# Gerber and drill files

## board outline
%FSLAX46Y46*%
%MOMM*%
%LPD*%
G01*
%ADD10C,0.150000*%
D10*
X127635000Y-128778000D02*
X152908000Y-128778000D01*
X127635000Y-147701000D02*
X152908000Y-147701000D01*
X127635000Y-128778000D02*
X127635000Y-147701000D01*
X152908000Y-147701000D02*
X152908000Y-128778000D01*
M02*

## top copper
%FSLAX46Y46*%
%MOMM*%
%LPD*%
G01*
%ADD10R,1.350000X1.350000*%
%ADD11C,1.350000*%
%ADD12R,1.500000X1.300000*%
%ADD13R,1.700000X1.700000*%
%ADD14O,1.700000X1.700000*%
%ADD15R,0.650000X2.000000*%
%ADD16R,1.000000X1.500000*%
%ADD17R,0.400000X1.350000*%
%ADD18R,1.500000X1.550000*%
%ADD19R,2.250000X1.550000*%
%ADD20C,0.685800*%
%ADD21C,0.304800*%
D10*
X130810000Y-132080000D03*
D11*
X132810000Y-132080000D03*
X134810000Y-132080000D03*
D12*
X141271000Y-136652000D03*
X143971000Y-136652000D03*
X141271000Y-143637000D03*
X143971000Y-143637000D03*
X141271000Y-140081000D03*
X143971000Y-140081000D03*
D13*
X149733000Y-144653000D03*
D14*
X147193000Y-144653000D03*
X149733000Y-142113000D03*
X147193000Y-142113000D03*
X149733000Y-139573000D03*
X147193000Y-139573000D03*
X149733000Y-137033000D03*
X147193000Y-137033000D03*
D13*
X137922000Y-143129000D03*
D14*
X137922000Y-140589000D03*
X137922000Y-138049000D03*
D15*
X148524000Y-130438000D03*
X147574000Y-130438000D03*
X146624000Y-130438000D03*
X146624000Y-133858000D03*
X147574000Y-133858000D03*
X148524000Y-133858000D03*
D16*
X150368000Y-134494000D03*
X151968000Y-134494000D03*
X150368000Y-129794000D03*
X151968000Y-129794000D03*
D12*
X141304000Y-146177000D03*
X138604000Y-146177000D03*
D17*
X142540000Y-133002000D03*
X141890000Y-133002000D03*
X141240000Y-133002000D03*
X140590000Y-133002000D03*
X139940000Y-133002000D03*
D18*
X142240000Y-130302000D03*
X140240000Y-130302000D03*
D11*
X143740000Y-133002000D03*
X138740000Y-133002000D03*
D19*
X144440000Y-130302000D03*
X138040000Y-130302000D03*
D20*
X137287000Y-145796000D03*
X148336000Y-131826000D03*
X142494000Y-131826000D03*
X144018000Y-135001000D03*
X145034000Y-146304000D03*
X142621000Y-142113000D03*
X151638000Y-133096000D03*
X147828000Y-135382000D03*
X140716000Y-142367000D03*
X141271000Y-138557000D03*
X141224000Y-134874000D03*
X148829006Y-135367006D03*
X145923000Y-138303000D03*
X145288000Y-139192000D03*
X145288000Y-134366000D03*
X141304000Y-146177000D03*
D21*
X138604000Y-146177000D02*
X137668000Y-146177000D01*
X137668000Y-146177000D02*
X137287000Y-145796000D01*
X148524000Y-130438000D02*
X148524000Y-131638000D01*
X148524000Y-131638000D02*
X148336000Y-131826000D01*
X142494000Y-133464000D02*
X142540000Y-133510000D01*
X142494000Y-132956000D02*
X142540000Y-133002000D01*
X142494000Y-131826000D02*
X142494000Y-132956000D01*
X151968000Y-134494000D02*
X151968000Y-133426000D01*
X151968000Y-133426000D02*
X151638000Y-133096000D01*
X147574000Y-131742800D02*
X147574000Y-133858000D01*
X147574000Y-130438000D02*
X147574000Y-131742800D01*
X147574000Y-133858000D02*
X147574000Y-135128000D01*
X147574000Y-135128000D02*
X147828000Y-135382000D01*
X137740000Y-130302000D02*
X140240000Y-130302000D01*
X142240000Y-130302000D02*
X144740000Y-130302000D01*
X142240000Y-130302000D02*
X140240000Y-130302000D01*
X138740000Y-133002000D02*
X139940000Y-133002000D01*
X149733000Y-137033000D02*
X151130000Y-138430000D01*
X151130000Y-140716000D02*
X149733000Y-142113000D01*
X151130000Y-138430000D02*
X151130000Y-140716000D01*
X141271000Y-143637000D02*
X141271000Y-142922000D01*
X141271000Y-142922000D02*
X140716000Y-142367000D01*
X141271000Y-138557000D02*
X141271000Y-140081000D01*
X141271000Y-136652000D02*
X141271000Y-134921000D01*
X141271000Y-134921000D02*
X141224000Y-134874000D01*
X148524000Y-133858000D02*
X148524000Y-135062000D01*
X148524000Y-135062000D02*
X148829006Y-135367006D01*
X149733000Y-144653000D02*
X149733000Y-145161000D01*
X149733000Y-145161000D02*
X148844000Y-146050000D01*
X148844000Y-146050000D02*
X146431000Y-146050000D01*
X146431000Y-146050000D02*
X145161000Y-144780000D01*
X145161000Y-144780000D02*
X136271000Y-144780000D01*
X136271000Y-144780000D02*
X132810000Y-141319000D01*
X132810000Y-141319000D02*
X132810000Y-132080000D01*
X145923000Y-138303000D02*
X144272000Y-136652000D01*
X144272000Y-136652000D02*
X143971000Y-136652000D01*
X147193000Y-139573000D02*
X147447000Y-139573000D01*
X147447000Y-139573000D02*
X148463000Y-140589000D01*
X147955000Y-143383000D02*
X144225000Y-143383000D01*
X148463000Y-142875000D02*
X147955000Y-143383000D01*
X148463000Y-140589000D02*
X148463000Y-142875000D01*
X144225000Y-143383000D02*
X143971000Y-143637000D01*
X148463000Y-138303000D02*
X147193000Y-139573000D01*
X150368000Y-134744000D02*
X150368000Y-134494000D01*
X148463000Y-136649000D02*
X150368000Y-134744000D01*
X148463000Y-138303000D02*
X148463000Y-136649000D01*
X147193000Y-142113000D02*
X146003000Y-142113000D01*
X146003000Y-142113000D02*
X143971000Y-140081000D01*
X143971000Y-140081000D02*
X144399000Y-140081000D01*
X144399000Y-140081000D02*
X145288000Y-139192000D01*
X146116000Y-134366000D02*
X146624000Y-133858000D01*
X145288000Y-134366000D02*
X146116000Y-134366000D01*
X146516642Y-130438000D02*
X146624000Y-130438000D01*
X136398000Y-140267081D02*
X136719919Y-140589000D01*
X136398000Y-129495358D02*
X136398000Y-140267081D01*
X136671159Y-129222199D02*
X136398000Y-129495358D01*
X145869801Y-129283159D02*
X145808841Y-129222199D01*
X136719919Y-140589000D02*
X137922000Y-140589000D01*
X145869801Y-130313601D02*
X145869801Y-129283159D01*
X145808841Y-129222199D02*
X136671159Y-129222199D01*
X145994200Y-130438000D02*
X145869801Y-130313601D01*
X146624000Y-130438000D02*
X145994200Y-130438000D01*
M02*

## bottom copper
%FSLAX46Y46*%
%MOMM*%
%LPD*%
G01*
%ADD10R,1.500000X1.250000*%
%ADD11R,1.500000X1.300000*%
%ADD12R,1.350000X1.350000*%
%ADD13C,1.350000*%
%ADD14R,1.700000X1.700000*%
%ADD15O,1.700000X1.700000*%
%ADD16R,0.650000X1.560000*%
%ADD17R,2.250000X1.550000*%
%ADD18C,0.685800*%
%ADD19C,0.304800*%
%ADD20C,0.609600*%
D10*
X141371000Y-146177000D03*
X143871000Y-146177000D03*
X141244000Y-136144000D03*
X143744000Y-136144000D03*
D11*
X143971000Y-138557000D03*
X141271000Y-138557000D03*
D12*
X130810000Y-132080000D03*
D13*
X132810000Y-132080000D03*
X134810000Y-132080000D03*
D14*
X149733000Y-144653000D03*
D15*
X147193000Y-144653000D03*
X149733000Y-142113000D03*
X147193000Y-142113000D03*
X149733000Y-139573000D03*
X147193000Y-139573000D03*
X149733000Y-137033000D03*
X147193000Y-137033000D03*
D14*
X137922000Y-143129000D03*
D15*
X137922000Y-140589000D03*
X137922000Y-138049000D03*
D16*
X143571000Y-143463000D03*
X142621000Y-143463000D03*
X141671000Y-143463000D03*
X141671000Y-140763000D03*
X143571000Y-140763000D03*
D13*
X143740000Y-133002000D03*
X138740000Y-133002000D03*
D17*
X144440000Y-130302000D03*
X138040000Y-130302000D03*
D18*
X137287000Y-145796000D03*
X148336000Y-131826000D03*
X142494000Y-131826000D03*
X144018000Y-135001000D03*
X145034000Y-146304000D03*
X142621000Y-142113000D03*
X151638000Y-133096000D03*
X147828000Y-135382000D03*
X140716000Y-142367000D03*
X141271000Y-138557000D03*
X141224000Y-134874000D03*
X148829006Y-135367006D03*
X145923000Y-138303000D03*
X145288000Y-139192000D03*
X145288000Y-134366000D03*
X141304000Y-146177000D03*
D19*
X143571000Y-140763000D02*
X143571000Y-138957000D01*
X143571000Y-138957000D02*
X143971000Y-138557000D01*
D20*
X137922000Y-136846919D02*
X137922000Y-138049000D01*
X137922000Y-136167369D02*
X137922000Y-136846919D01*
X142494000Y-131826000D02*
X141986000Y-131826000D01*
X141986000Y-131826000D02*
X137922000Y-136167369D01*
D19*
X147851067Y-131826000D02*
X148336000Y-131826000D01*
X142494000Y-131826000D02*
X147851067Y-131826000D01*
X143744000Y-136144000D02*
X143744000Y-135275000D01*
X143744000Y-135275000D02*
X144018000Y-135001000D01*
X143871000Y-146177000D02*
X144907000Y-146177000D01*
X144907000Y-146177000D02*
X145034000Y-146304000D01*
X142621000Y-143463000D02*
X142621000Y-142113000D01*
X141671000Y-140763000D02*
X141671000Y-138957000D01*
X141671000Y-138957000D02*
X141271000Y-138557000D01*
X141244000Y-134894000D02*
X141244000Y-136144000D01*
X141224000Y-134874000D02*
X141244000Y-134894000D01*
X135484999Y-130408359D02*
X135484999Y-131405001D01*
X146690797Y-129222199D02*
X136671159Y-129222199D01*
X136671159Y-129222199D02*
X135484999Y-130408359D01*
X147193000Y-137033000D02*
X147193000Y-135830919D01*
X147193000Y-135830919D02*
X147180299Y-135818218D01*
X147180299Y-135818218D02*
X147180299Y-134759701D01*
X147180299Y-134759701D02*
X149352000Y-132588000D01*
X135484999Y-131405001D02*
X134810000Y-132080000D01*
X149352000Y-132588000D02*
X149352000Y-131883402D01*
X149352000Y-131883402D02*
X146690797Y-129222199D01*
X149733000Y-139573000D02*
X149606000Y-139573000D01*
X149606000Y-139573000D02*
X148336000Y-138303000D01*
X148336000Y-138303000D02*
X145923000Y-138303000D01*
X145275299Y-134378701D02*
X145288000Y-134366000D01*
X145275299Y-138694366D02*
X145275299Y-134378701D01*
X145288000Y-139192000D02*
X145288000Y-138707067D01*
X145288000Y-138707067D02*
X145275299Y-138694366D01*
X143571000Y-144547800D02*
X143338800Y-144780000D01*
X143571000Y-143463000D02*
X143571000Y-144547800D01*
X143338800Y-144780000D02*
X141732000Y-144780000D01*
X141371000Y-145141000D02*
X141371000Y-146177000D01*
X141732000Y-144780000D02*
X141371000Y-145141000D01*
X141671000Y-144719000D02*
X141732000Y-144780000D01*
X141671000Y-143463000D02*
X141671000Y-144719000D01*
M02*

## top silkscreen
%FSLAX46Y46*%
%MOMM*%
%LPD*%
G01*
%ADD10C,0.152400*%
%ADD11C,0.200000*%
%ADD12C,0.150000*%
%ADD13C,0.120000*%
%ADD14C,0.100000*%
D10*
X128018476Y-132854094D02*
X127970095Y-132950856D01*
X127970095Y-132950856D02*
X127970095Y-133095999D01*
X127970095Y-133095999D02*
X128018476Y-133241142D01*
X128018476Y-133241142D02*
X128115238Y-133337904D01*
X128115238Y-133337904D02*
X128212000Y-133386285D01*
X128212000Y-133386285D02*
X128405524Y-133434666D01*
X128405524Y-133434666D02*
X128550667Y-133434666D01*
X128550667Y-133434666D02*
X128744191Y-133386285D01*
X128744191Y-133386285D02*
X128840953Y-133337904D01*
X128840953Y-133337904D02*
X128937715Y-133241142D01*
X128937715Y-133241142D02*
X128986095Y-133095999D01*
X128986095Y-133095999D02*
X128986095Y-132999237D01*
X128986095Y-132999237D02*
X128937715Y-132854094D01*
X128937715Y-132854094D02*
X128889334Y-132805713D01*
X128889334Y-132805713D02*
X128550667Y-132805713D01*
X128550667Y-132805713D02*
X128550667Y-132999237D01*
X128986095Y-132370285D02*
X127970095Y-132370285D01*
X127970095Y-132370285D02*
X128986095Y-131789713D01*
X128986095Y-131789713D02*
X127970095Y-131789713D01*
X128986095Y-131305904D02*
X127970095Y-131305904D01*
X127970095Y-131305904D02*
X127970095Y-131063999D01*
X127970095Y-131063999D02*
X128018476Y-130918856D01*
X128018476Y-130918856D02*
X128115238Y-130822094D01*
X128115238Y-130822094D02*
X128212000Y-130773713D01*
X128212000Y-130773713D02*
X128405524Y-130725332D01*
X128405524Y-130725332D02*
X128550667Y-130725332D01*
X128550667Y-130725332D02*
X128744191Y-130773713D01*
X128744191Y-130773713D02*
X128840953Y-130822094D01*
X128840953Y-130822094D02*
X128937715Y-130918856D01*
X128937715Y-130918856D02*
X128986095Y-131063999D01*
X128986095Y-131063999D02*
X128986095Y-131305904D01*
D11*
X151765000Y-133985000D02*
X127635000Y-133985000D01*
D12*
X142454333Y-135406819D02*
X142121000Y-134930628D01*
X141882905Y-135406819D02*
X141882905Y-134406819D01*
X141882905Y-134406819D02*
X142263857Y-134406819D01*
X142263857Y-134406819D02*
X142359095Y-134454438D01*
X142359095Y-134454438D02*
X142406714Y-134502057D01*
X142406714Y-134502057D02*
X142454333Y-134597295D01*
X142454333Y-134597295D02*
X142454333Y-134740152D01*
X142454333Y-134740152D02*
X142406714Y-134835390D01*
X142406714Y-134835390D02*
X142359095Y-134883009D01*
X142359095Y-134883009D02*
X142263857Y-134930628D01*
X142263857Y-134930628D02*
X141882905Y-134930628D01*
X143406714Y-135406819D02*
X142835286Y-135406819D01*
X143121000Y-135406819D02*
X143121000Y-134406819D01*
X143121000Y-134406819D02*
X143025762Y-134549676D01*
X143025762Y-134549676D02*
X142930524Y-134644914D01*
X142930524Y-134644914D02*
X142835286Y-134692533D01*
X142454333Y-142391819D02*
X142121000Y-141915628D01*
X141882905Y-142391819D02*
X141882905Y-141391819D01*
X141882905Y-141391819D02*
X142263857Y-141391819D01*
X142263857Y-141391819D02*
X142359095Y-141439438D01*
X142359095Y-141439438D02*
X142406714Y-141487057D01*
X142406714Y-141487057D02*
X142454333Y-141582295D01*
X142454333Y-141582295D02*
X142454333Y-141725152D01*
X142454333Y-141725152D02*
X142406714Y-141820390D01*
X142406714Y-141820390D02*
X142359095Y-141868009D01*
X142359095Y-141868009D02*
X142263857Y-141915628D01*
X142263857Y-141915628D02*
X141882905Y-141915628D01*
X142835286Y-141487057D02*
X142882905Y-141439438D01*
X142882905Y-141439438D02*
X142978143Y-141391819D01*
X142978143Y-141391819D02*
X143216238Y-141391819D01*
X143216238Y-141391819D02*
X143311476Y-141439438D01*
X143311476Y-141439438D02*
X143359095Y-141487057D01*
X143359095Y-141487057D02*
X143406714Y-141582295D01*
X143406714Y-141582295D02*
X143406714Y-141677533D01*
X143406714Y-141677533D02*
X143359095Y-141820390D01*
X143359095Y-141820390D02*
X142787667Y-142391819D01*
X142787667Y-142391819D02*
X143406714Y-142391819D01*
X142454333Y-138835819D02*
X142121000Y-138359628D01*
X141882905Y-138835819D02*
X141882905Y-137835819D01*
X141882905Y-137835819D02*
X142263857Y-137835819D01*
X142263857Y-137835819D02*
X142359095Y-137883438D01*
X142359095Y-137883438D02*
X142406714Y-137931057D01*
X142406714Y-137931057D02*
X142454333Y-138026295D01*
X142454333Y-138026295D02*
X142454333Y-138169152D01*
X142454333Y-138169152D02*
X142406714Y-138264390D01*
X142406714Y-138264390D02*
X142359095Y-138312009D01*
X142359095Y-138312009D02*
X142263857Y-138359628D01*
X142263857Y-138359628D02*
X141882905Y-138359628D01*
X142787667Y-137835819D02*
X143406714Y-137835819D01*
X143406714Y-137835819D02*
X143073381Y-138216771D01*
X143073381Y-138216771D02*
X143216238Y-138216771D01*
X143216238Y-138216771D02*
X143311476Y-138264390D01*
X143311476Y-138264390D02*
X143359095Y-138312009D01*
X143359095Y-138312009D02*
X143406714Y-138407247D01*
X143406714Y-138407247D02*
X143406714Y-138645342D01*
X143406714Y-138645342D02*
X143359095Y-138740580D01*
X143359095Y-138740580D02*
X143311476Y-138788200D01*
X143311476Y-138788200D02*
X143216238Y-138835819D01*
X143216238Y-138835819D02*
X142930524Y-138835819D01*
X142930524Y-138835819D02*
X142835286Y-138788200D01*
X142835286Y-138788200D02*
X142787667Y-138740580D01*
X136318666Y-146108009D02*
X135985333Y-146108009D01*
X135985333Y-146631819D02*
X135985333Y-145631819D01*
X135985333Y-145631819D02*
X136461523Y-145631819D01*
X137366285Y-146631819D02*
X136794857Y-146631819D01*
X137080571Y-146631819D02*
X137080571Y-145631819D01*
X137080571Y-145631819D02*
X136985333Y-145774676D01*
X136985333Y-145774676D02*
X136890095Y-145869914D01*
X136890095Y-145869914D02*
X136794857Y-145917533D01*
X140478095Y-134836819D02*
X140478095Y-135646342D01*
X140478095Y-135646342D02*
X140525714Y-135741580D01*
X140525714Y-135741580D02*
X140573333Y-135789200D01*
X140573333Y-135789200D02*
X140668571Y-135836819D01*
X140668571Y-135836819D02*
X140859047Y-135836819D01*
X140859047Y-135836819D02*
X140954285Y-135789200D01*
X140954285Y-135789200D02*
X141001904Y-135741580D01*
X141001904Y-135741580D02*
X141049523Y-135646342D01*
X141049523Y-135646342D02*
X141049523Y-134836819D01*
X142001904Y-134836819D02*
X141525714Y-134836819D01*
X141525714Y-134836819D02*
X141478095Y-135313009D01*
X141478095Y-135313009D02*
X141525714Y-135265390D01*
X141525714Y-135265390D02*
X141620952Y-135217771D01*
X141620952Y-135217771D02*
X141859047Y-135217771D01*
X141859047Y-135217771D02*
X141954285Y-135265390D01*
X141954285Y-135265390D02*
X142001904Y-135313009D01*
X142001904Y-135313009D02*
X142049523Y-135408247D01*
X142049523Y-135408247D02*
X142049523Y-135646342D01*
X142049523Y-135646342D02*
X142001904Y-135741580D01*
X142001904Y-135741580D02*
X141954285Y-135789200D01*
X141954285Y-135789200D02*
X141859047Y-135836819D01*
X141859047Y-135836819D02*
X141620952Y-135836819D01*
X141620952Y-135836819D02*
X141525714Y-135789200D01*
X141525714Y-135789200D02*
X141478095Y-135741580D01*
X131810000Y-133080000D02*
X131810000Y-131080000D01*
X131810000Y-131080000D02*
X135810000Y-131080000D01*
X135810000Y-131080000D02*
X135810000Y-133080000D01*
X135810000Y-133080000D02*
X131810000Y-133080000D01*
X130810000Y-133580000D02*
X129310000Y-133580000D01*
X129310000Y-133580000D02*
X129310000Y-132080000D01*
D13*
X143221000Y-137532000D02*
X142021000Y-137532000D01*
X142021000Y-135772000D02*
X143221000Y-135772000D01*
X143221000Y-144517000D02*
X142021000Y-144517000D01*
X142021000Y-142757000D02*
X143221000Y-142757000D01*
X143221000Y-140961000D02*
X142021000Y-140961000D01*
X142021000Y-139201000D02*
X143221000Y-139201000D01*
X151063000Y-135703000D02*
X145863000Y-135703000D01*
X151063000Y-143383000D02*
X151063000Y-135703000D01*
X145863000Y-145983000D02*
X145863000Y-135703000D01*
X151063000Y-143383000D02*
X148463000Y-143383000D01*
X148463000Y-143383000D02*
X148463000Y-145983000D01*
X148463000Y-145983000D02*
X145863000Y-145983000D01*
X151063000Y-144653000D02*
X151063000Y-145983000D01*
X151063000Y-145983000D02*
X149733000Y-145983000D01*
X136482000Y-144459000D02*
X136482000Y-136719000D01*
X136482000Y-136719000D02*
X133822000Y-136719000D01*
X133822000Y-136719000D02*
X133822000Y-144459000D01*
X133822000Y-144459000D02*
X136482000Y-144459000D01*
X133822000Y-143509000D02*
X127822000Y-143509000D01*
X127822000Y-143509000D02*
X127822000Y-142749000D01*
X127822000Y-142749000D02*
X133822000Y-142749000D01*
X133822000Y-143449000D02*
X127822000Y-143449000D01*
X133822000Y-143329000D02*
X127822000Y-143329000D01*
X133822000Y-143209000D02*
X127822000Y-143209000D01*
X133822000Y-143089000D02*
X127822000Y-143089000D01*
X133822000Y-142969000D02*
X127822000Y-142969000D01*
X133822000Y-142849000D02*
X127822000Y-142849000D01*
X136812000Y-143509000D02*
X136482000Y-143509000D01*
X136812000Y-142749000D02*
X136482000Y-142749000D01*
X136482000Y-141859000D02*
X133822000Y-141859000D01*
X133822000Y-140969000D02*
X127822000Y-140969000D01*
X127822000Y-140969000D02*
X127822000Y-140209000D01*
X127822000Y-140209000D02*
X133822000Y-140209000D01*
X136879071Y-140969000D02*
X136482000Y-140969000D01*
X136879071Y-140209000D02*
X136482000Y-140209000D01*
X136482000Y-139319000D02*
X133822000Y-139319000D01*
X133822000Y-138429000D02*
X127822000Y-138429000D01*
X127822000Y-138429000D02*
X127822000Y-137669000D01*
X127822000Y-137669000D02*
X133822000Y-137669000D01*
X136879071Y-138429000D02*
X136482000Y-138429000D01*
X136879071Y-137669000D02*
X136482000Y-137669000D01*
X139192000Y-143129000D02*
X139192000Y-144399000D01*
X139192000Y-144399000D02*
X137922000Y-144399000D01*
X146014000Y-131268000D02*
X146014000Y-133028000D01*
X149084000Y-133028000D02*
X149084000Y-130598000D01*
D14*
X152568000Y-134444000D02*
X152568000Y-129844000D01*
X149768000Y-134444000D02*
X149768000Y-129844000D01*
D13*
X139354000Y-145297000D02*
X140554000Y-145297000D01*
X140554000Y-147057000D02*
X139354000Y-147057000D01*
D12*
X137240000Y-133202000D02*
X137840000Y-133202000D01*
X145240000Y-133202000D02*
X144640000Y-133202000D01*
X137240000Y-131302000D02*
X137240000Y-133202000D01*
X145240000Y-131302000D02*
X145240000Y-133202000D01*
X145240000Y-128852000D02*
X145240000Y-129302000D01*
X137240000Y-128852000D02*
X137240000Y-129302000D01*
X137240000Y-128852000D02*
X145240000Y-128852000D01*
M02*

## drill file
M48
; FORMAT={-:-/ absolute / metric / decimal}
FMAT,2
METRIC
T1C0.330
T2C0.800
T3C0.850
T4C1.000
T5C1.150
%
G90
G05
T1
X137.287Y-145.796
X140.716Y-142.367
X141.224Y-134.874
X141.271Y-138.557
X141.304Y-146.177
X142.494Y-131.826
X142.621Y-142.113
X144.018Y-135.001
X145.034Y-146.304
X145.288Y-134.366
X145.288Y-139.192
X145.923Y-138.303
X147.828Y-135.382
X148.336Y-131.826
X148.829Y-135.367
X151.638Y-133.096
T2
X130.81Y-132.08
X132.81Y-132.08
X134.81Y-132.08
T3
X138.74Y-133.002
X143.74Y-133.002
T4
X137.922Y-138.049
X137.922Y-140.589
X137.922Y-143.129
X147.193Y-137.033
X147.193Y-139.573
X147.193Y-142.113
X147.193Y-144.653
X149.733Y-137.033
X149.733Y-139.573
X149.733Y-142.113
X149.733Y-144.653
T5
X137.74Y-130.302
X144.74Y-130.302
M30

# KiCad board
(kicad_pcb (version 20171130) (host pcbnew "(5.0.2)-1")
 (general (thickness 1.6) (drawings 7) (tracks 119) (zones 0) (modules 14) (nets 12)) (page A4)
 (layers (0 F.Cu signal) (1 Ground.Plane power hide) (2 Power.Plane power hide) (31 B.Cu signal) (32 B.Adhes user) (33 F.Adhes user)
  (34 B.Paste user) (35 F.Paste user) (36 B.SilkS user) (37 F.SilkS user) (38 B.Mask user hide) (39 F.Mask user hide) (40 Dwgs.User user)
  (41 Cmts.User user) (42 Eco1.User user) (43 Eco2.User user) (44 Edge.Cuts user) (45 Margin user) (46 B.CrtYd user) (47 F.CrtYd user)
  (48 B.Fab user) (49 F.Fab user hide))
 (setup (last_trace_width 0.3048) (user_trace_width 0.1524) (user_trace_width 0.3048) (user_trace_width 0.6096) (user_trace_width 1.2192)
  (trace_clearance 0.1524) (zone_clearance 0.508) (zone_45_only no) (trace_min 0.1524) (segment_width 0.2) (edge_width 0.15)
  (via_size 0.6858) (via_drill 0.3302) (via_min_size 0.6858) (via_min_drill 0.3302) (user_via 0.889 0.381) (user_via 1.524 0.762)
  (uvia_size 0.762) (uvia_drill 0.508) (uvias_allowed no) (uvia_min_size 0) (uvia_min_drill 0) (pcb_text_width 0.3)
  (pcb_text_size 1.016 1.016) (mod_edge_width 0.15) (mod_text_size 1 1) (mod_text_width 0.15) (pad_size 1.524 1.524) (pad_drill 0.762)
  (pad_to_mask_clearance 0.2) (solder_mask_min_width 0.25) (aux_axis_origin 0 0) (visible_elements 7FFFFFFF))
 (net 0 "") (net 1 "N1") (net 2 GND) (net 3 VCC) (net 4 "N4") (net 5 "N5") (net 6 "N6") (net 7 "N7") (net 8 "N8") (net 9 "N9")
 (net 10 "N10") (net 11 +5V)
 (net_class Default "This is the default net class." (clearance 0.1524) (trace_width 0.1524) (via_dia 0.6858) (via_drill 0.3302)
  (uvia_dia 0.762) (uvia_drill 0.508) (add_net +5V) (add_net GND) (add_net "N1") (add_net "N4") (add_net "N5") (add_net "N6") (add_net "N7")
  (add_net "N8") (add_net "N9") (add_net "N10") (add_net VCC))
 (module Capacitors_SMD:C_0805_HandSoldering (layer B.Cu) (at 142.621 146.177)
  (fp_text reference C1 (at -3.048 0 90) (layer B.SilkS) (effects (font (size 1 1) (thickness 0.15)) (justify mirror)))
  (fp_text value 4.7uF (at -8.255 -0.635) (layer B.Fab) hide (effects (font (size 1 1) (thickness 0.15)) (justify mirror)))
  (pad 1 smd rect (at -1.25 0) (size 1.5 1.25) (layers B.Cu B.Paste B.Mask) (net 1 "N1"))
  (pad 2 smd rect (at 1.25 0) (size 1.5 1.25) (layers B.Cu B.Paste B.Mask) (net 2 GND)))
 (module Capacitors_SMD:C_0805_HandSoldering (layer B.Cu) (at 142.494 136.144)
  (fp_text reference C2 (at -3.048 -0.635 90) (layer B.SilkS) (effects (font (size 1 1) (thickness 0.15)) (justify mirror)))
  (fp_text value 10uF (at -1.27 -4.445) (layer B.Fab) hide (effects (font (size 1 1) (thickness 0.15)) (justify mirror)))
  (pad 1 smd rect (at -1.25 0) (size 1.5 1.25) (layers B.Cu B.Paste B.Mask) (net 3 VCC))
  (pad 2 smd rect (at 1.25 0) (size 1.5 1.25) (layers B.Cu B.Paste B.Mask) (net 2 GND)))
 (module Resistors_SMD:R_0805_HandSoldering (layer B.Cu) (at 142.621 138.557 180)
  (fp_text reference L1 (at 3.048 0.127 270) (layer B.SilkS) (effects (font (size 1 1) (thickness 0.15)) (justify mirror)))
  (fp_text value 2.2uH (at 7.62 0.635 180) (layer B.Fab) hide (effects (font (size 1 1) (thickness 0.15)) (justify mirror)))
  (pad 1 smd rect (at -1.35 0 180) (size 1.5 1.3) (layers B.Cu B.Paste B.Mask) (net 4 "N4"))
  (pad 2 smd rect (at 1.35 0 180) (size 1.5 1.3) (layers B.Cu B.Paste B.Mask) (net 3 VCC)))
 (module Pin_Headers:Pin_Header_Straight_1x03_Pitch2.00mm (layer F.Cu) (at 130.81 132.08 90)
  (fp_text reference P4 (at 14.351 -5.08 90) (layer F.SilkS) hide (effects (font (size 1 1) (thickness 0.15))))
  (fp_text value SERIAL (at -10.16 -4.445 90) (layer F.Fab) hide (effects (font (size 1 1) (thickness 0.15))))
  (fp_line (start -1 1) (end 1 1) (layer F.SilkS) (width 0.15)) (fp_line (start 1 1) (end 1 5) (layer F.SilkS) (width 0.15))
  (fp_line (start 1 5) (end -1 5) (layer F.SilkS) (width 0.15))
  (fp_line (start -1 5) (end -1 1) (layer F.SilkS) (width 0.15))
  (fp_line (start -1.5 0) (end -1.5 -1.5) (layer F.SilkS) (width 0.15))
  (fp_line (start -1.5 -1.5) (end 0 -1.5) (layer F.SilkS) (width 0.15))
  (pad 1 thru_hole rect (at 0 0 90) (size 1.35 1.35) (drill 0.8) (layers *.Cu *.Mask) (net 2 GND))
  (pad 2 thru_hole circle (at 0 2 90) (size 1.35 1.35) (drill 0.8) (layers *.Cu *.Mask) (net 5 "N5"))
  (pad 3 thru_hole circle (at 0 4 90) (size 1.35 1.35) (drill 0.8) (layers *.Cu *.Mask) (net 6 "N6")))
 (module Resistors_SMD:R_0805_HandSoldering (layer F.Cu) (at 142.621 136.652)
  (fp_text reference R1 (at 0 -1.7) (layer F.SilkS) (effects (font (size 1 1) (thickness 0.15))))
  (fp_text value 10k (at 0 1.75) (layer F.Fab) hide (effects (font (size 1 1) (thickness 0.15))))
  (fp_line (start 0.6 0.88) (end -0.6 0.88) (layer F.SilkS) (width 0.12))
  (fp_line (start -0.6 -0.88) (end 0.6 -0.88) (layer F.SilkS) (width 0.12))
  (pad 1 smd rect (at -1.35 0) (size 1.5 1.3) (layers F.Cu F.Paste F.Mask) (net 3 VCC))
  (pad 2 smd rect (at 1.35 0) (size 1.5 1.3) (layers F.Cu F.Paste F.Mask) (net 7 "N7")))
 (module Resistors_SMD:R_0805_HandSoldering (layer F.Cu) (at 142.621 143.637)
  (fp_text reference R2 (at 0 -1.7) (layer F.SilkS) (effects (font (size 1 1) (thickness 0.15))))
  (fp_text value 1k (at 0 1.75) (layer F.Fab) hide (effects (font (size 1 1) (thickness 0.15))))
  (fp_line (start 0.6 0.88) (end -0.6 0.88) (layer F.SilkS) (width 0.12))
  (fp_line (start -0.6 -0.88) (end 0.6 -0.88) (layer F.SilkS) (width 0.12))
  (pad 1 smd rect (at -1.35 0) (size 1.5 1.3) (layers F.Cu F.Paste F.Mask) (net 3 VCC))
  (pad 2 smd rect (at 1.35 0) (size 1.5 1.3) (layers F.Cu F.Paste F.Mask) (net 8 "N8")))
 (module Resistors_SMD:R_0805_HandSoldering (layer F.Cu) (at 142.621 140.081)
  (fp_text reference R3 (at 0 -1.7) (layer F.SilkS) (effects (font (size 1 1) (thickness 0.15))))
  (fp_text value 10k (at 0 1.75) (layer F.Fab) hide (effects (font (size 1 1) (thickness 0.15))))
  (fp_line (start 0.6 0.88) (end -0.6 0.88) (layer F.SilkS) (width 0.12))
  (fp_line (start -0.6 -0.88) (end 0.6 -0.88) (layer F.SilkS) (width 0.12))
  (pad 1 smd rect (at -1.35 0) (size 1.5 1.3) (layers F.Cu F.Paste F.Mask) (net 3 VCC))
  (pad 2 smd rect (at 1.35 0) (size 1.5 1.3) (layers F.Cu F.Paste F.Mask) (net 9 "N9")))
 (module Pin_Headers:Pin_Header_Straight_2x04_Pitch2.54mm (layer F.Cu) (at 149.733 144.653 180)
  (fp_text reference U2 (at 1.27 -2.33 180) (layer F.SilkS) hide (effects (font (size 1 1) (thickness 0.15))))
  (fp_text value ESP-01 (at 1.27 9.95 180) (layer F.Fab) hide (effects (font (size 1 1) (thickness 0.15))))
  (fp_line (start -1.33 8.95) (end 3.87 8.95) (layer F.SilkS) (width 0.12))
  (fp_line (start -1.33 1.27) (end -1.33 8.95) (layer F.SilkS) (width 0.12))
  (fp_line (start 3.87 -1.33) (end 3.87 8.95) (layer F.SilkS) (width 0.12))
  (fp_line (start -1.33 1.27) (end 1.27 1.27) (layer F.SilkS) (width 0.12))
  (fp_line (start 1.27 1.27) (end 1.27 -1.33) (layer F.SilkS) (width 0.12))
  (fp_line (start 1.27 -1.33) (end 3.87 -1.33) (layer F.SilkS) (width 0.12))
  (fp_line (start -1.33 0) (end -1.33 -1.33) (layer F.SilkS) (width 0.12))
  (fp_line (start -1.33 -1.33) (end 0 -1.33) (layer F.SilkS) (width 0.12))
  (pad 1 thru_hole rect (at 0 0 180) (size 1.7 1.7) (drill 1) (layers *.Cu *.Mask) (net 5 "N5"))
  (pad 2 thru_hole oval (at 2.54 0 180) (size 1.7 1.7) (drill 1) (layers *.Cu *.Mask) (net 2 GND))
  (pad 3 thru_hole oval (at 0 2.54 180) (size 1.7 1.7) (drill 1) (layers *.Cu *.Mask) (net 3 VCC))
  (pad 4 thru_hole oval (at 2.54 2.54 180) (size 1.7 1.7) (drill 1) (layers *.Cu *.Mask) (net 9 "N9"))
  (pad 5 thru_hole oval (at 0 5.08 180) (size 1.7 1.7) (drill 1) (layers *.Cu *.Mask) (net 7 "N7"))
  (pad 6 thru_hole oval (at 2.54 5.08 180) (size 1.7 1.7) (drill 1) (layers *.Cu *.Mask) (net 8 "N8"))
  (pad 7 thru_hole oval (at 0 7.62 180) (size 1.7 1.7) (drill 1) (layers *.Cu *.Mask) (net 3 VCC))
  (pad 8 thru_hole oval (at 2.54 7.62 180) (size 1.7 1.7) (drill 1) (layers *.Cu *.Mask) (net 6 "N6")))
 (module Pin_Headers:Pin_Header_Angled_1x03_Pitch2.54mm (layer F.Cu) (at 137.922 143.129 180)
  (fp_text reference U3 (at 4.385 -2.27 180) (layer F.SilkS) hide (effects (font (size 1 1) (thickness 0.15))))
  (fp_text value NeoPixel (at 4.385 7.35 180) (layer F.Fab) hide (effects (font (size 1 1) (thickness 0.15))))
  (fp_line (start 1.44 -1.33) (end 1.44 6.41) (layer F.SilkS) (width 0.12))
  (fp_line (start 1.44 6.41) (end 4.1 6.41) (layer F.SilkS) (width 0.12))
  (fp_line (start 4.1 6.41) (end 4.1 -1.33) (layer F.SilkS) (width 0.12))
  (fp_line (start 4.1 -1.33) (end 1.44 -1.33) (layer F.SilkS) (width 0.12))
  (fp_line (start 4.1 -0.38) (end 10.1 -0.38) (layer F.SilkS) (width 0.12))
  (fp_line (start 10.1 -0.38) (end 10.1 0.38) (layer F.SilkS) (width 0.12))
  (fp_line (start 10.1 0.38) (end 4.1 0.38) (layer F.SilkS) (width 0.12))
  (fp_line (start 4.1 -0.32) (end 10.1 -0.32) (layer F.SilkS) (width 0.12))
  (fp_line (start 4.1 -0.2) (end 10.1 -0.2) (layer F.SilkS) (width 0.12))
  (fp_line (start 4.1 -0.08) (end 10.1 -0.08) (layer F.SilkS) (width 0.12))
  (fp_line (start 4.1 0.04) (end 10.1 0.04) (layer F.SilkS) (width 0.12))
  (fp_line (start 4.1 0.16) (end 10.1 0.16) (layer F.SilkS) (width 0.12))
  (fp_line (start 4.1 0.28) (end 10.1 0.28) (layer F.SilkS) (width 0.12))
  (fp_line (start 1.11 -0.38) (end 1.44 -0.38) (layer F.SilkS) (width 0.12))
  (fp_line (start 1.11 0.38) (end 1.44 0.38) (layer F.SilkS) (width 0.12))
  (fp_line (start 1.44 1.27) (end 4.1 1.27) (layer F.SilkS) (width 0.12))
  (fp_line (start 4.1 2.16) (end 10.1 2.16) (layer F.SilkS) (width 0.12))
  (fp_line (start 10.1 2.16) (end 10.1 2.92) (layer F.SilkS) (width 0.12))
  (fp_line (start 10.1 2.92) (end 4.1 2.92) (layer F.SilkS) (width 0.12))
  (fp_line (start 1.042929 2.16) (end 1.44 2.16) (layer F.SilkS) (width 0.12))
  (fp_line (start 1.042929 2.92) (end 1.44 2.92) (layer F.SilkS) (width 0.12))
  (fp_line (start 1.44 3.81) (end 4.1 3.81) (layer F.SilkS) (width 0.12))
  (fp_line (start 4.1 4.7) (end 10.1 4.7) (layer F.SilkS) (width 0.12))
  (fp_line (start 10.1 4.7) (end 10.1 5.46) (layer F.SilkS) (width 0.12))
  (fp_line (start 10.1 5.46) (end 4.1 5.46) (layer F.SilkS) (width 0.12))
  (fp_line (start 1.042929 4.7) (end 1.44 4.7) (layer F.SilkS) (width 0.12))
  (fp_line (start 1.042929 5.46) (end 1.44 5.46) (layer F.SilkS) (width 0.12))
  (fp_line (start -1.27 0) (end -1.27 -1.27) (layer F.SilkS) (width 0.12))
  (fp_line (start -1.27 -1.27) (end 0 -1.27) (layer F.SilkS) (width 0.12))
  (pad 1 thru_hole rect (at 0 0 180) (size 1.7 1.7) (drill 1) (layers *.Cu *.Mask) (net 2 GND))
  (pad 2 thru_hole oval (at 0 2.54 180) (size 1.7 1.7) (drill 1) (layers *.Cu *.Mask) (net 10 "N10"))
  (pad 3 thru_hole oval (at 0 5.08 180) (size 1.7 1.7) (drill 1) (layers *.Cu *.Mask) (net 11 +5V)))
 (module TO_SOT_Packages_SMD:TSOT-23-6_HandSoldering (layer F.Cu) (at 147.574 132.148 270)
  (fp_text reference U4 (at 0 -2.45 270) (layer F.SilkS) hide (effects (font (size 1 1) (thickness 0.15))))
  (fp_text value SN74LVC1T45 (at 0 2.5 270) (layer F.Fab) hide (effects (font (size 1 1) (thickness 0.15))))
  (fp_line (start -0.88 1.56) (end 0.88 1.56) (layer F.SilkS) (width 0.12))
  (fp_line (start 0.88 -1.51) (end -1.55 -1.51) (layer F.SilkS) (width 0.12))
  (pad 1 smd rect (at -1.71 -0.95 270) (size 2 0.65) (layers F.Cu F.Paste F.Mask) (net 11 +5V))
  (pad 2 smd rect (at -1.71 0 270) (size 2 0.65) (layers F.Cu F.Paste F.Mask) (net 2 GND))
  (pad 3 smd rect (at -1.71 0.95 270) (size 2 0.65) (layers F.Cu F.Paste F.Mask) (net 10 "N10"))
  (pad 4 smd rect (at 1.71 0.95 270) (size 2 0.65) (layers F.Cu F.Paste F.Mask) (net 9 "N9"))
  (pad 5 smd rect (at 1.71 0 270) (size 2 0.65) (layers F.Cu F.Paste F.Mask) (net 2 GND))
  (pad 6 smd rect (at 1.71 -0.95 270) (size 2 0.65) (layers F.Cu F.Paste F.Mask) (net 3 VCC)))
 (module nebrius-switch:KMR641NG (layer F.Cu) (at 151.168 132.144 90)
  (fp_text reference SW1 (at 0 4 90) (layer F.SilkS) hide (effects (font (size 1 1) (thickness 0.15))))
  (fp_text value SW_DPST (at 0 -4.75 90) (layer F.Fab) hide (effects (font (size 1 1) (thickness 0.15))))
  (fp_line (start -2.3 1.4) (end 2.3 1.4) (layer F.SilkS) (width 0.1))
  (fp_line (start -2.3 -1.4) (end 2.3 -1.4) (layer F.SilkS) (width 0.1))
  (pad 1 smd rect (at -2.35 -0.8 90) (size 1.5 1) (layers F.Cu F.Paste F.Mask) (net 8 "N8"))
  (pad 2 smd rect (at -2.35 0.8 90) (size 1.5 1) (layers F.Cu F.Paste F.Mask) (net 2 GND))
  (pad 3 smd rect (at 2.35 -0.8 90) (size 1.5 1) (layers F.Cu F.Paste F.Mask))
  (pad 4 smd rect (at 2.35 0.8 90) (size 1.5 1) (layers F.Cu F.Paste F.Mask)))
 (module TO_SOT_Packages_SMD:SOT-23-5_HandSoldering (layer B.Cu) (at 142.621 142.113 90)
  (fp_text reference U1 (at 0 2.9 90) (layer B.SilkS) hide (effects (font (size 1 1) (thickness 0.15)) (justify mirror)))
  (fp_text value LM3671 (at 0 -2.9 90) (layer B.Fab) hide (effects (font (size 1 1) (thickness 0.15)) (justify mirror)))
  (pad 1 smd rect (at -1.35 0.95 90) (size 1.56 0.65) (layers B.Cu B.Paste B.Mask) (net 1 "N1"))
  (pad 2 smd rect (at -1.35 0 90) (size 1.56 0.65) (layers B.Cu B.Paste B.Mask) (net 2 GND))
  (pad 3 smd rect (at -1.35 -0.95 90) (size 1.56 0.65) (layers B.Cu B.Paste B.Mask) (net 1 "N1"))
  (pad 4 smd rect (at 1.35 -0.95 90) (size 1.56 0.65) (layers B.Cu B.Paste B.Mask) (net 3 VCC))
  (pad 5 smd rect (at 1.35 0.95 90) (size 1.56 0.65) (layers B.Cu B.Paste B.Mask) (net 4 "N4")))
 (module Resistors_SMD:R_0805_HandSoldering (layer F.Cu) (at 139.954 146.177 180)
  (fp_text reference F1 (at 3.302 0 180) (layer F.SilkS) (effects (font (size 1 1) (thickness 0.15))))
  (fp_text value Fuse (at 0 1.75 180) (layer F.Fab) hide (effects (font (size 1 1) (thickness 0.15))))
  (fp_line (start 0.6 0.88) (end -0.6 0.88) (layer F.SilkS) (width 0.12))
  (fp_line (start -0.6 -0.88) (end 0.6 -0.88) (layer F.SilkS) (width 0.12))
  (pad 1 smd rect (at -1.35 0 180) (size 1.5 1.3) (layers F.Cu F.Paste F.Mask) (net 1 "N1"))
  (pad 2 smd rect (at 1.35 0 180) (size 1.5 1.3) (layers F.Cu F.Paste F.Mask) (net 11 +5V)))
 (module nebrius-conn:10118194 (layer F.Cu) (at 141.24 130.302 180)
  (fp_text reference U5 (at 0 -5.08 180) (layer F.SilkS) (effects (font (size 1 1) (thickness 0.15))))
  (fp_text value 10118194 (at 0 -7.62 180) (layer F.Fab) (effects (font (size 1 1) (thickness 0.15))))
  (fp_line (start 4 -2.9) (end 3.4 -2.9) (layer F.SilkS) (width 0.15))
  (fp_line (start -4 -2.9) (end -3.4 -2.9) (layer F.SilkS) (width 0.15))
  (fp_line (start 4 -1) (end 4 -2.9) (layer F.SilkS) (width 0.15))
  (fp_line (start -4 -1) (end -4 -2.9) (layer F.SilkS) (width 0.15))
  (fp_line (start -4 1.45) (end -4 1) (layer F.SilkS) (width 0.15))
  (fp_line (start 4 1.45) (end 4 1) (layer F.SilkS) (width 0.15))
  (fp_line (start 4 1.45) (end -4 1.45) (layer F.SilkS) (width 0.15))
  (pad 1 smd rect (at -1.3 -2.7 180) (size 0.4 1.35) (layers F.Cu F.Paste F.Mask) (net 11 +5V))
  (pad 2 smd rect (at -0.65 -2.7 180) (size 0.4 1.35) (layers F.Cu F.Paste F.Mask))
  (pad 3 smd rect (at 0 -2.7 180) (size 0.4 1.35) (layers F.Cu F.Paste F.Mask))
  (pad 4 smd rect (at 0.65 -2.7 180) (size 0.4 1.35) (layers F.Cu F.Paste F.Mask))
  (pad 5 smd rect (at 1.3 -2.7 180) (size 0.4 1.35) (layers F.Cu F.Paste F.Mask) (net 2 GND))
  (pad 5 smd rect (at -1 0 180) (size 1.5 1.55) (layers F.Cu F.Paste F.Mask) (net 2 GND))
  (pad 5 smd rect (at 1 0 180) (size 1.5 1.55) (layers F.Cu F.Paste F.Mask) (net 2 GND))
  (pad 5 thru_hole circle (at -2.5 -2.7 180) (size 1.35 1.35) (drill 0.85) (layers *.Cu *.Mask) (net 2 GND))
  (pad 5 thru_hole circle (at 2.5 -2.7 180) (size 1.35 1.35) (drill 0.85) (layers *.Cu *.Mask) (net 2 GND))
  (pad 5 thru_hole rect (at -3.5 0 180) (size 2.25 1.55) (drill 1.15 (offset 0.3 0)) (layers *.Cu *.Mask) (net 2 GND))
  (pad 5 thru_hole rect (at 3.5 0 180) (size 2.25 1.55) (drill 1.15 (offset -0.3 0)) (layers *.Cu *.Mask) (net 2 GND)))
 (gr_line (start 127.635 128.778) (end 152.908 128.778) (angle 90) (layer Edge.Cuts) (width 0.15))
 (gr_line (start 127.635 147.701) (end 152.908 147.701) (angle 90) (layer Edge.Cuts) (width 0.15))
 (gr_line (start 127.635 128.778) (end 127.635 147.701) (angle 90) (layer Edge.Cuts) (width 0.15))
 (gr_line (start 152.908 147.701) (end 152.908 128.778) (angle 90) (layer Edge.Cuts) (width 0.15))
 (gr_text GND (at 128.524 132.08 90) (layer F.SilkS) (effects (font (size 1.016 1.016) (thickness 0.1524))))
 (gr_line (start 151.765 133.985) (end 127.635 133.985) (angle 90) (layer F.SilkS) (width 0.2))
 (segment (start 143.571 140.763) (end 143.571 138.957) (width 0.3048) (layer B.Cu) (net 4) (status 30))
 (segment (start 143.571 138.957) (end 143.971 138.557) (width 0.3048) (layer B.Cu) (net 4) (status 30))
 (segment (start 138.604 146.177) (end 137.668 146.177) (width 0.3048) (layer F.Cu) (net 11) (status 10))
 (via (at 137.287 145.796) (size 0.6858) (drill 0.3302) (layers F.Cu B.Cu) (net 11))
 (segment (start 137.668 146.177) (end 137.287 145.796) (width 0.3048) (layer F.Cu) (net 11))
 (via (at 148.336 131.826) (size 0.6858) (drill 0.3302) (layers F.Cu B.Cu) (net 11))
 (segment (start 148.524 130.438) (end 148.524 131.638) (width 0.3048) (layer F.Cu) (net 11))
 (segment (start 148.524 131.638) (end 148.336 131.826) (width 0.3048) (layer F.Cu) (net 11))
 (segment (start 142.494 133.464) (end 142.54 133.51) (width 0.3048) (layer F.Cu) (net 11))
 (via (at 142.494 131.826) (size 0.6858) (drill 0.3302) (layers F.Cu B.Cu) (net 11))
 (segment (start 137.922 136.846919) (end 137.922 138.049) (width 0.6096) (layer B.Cu) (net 11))
 (segment (start 137.922 136.167369) (end 137.922 136.846919) (width 0.6096) (layer B.Cu) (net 11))
 (segment (start 142.494 131.826) (end 141.986 131.826) (width 0.6096) (layer B.Cu) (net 11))
 (segment (start 141.986 131.826) (end 137.922 136.167369) (width 0.6096) (layer B.Cu) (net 11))
 (segment (start 147.851067 131.826) (end 148.336 131.826) (width 0.3048) (layer B.Cu) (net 11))
 (segment (start 142.494 131.826) (end 147.851067 131.826) (width 0.3048) (layer B.Cu) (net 11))
 (segment (start 142.494 132.956) (end 142.54 133.002) (width 0.3048) (layer F.Cu) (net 11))
 (segment (start 142.494 131.826) (end 142.494 132.956) (width 0.3048) (layer F.Cu) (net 11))
 (segment (start 143.744 136.144) (end 143.744 135.275) (width 0.3048) (layer B.Cu) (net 2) (status 10))
 (via (at 144.018 135.001) (size 0.6858) (drill 0.3302) (layers F.Cu B.Cu) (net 2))
 (segment (start 143.744 135.275) (end 144.018 135.001) (width 0.3048) (layer B.Cu) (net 2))
 (segment (start 143.871 146.177) (end 144.907 146.177) (width 0.3048) (layer B.Cu) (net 2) (status 10))
 (via (at 145.034 146.304) (size 0.6858) (drill 0.3302) (layers F.Cu B.Cu) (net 2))
 (segment (start 144.907 146.177) (end 145.034 146.304) (width 0.3048) (layer B.Cu) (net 2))
 (segment (start 142.621 143.463) (end 142.621 142.113) (width 0.3048) (layer B.Cu) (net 2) (status 10))
 (via (at 142.621 142.113) (size 0.6858) (drill 0.3302) (layers F.Cu B.Cu) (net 2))
 (via (at 151.638 133.096) (size 0.6858) (drill 0.3302) (layers F.Cu B.Cu) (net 2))
 (segment (start 151.968 134.494) (end 151.968 133.426) (width 0.3048) (layer F.Cu) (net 2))
 (segment (start 151.968 133.426) (end 151.638 133.096) (width 0.3048) (layer F.Cu) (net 2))
 (segment (start 147.574 131.7428) (end 147.574 133.858) (width 0.3048) (layer F.Cu) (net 2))
 (segment (start 147.574 130.438) (end 147.574 131.7428) (width 0.3048) (layer F.Cu) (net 2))
 (via (at 147.828 135.382) (size 0.6858) (drill 0.3302) (layers F.Cu B.Cu) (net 2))
 (segment (start 147.574 133.858) (end 147.574 135.128) (width 0.3048) (layer F.Cu) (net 2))
 (segment (start 147.574 135.128) (end 147.828 135.382) (width 0.3048) (layer F.Cu) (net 2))
 (segment (start 137.74 130.302) (end 140.24 130.302) (width 0.3048) (layer F.Cu) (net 2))
 (segment (start 142.24 130.302) (end 144.74 130.302) (width 0.3048) (layer F.Cu) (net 2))
 (segment (start 142.24 130.302) (end 140.24 130.302) (width 0.3048) (layer F.Cu) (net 2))
 (segment (start 138.74 133.002) (end 139.94 133.002) (width 0.3048) (layer F.Cu) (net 2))
 (segment (start 149.733 137.033) (end 151.13 138.43) (width 0.3048) (layer F.Cu) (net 3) (status 10))
 (segment (start 151.13 140.716) (end 149.733 142.113) (width 0.3048) (layer F.Cu) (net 3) (status 20))
 (segment (start 151.13 138.43) (end 151.13 140.716) (width 0.3048) (layer F.Cu) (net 3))
 (segment (start 141.271 143.637) (end 141.271 142.922) (width 0.3048) (layer F.Cu) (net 3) (status 10))
 (via (at 140.716 142.367) (size 0.6858) (drill 0.3302) (layers F.Cu B.Cu) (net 3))
 (segment (start 141.271 142.922) (end 140.716 142.367) (width 0.3048) (layer F.Cu) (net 3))
 (segment (start 141.671 140.763) (end 141.671 138.957) (width 0.3048) (layer B.Cu) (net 3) (status 30))
 (segment (start 141.671 138.957) (end 141.271 138.557) (width 0.3048) (layer B.Cu) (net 3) (status 30))
 (via (at 141.271 138.557) (size 0.6858) (drill 0.3302) (layers F.Cu B.Cu) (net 3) (status 30))
 (segment (start 141.271 138.557) (end 141.271 140.081) (width 0.3048) (layer F.Cu) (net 3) (status 20))
 (segment (start 141.271 136.652) (end 141.271 134.921) (width 0.3048) (layer F.Cu) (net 3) (status 10))
 (segment (start 141.244 134.894) (end 141.244 136.144) (width 0.3048) (layer B.Cu) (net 3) (status 20))
 (segment (start 141.224 134.874) (end 141.244 134.894) (width 0.3048) (layer B.Cu) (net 3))
 (via (at 141.224 134.874) (size 0.6858) (drill 0.3302) (layers F.Cu B.Cu) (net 3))
 (segment (start 141.271 134.921) (end 141.224 134.874) (width 0.3048) (layer F.Cu) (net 3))
 (via (at 148.829006 135.367006) (size 0.6858) (drill 0.3302) (layers F.Cu B.Cu) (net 3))
 (segment (start 148.524 133.858) (end 148.524 135.062) (width 0.3048) (layer F.Cu) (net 3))
 (segment (start 148.524 135.062) (end 148.829006 135.367006) (width 0.3048) (layer F.Cu) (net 3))
 (segment (start 149.733 144.653) (end 149.733 145.161) (width 0.3048) (layer F.Cu) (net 5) (status 30))
 (segment (start 149.733 145.161) (end 148.844 146.05) (width 0.3048) (layer F.Cu) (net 5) (status 10))
 (segment (start 148.844 146.05) (end 146.431 146.05) (width 0.3048) (layer F.Cu) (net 5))
 (segment (start 146.431 146.05) (end 145.161 144.78) (width 0.3048) (layer F.Cu) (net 5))
 (segment (start 145.161 144.78) (end 136.271 144.78) (width 0.3048) (layer F.Cu) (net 5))
 (segment (start 136.271 144.78) (end 132.81 141.319) (width 0.3048) (layer F.Cu) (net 5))
 (segment (start 132.81 141.319) (end 132.81 132.08) (width 0.3048) (layer F.Cu) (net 5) (status 20))
 (segment (start 135.484999 130.408359) (end 135.484999 131.405001) (width 0.3048) (layer B.Cu) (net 6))
 (segment (start 146.690797 129.222199) (end 136.671159 129.222199) (width 0.3048) (layer B.Cu) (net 6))
 (segment (start 136.671159 129.222199) (end 135.484999 130.408359) (width 0.3048) (layer B.Cu) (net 6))
 (segment (start 147.193 137.033) (end 147.193 135.830919) (width 0.3048) (layer B.Cu) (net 6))
 (segment (start 147.193 135.830919) (end 147.180299 135.818218) (width 0.3048) (layer B.Cu) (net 6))
 (segment (start 147.180299 135.818218) (end 147.180299 134.759701) (width 0.3048) (layer B.Cu) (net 6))
 (segment (start 147.180299 134.759701) (end 149.352 132.588) (width 0.3048) (layer B.Cu) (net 6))
 (segment (start 135.484999 131.405001) (end 134.81 132.08) (width 0.3048) (layer B.Cu) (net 6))
 (segment (start 149.352 132.588) (end 149.352 131.883402) (width 0.3048) (layer B.Cu) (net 6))
 (segment (start 149.352 131.883402) (end 146.690797 129.222199) (width 0.3048) (layer B.Cu) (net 6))
 (segment (start 149.733 139.573) (end 149.606 139.573) (width 0.3048) (layer B.Cu) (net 7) (status 30))
 (segment (start 149.606 139.573) (end 148.336 138.303) (width 0.3048) (layer B.Cu) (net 7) (status 10))
 (segment (start 148.336 138.303) (end 145.923 138.303) (width 0.3048) (layer B.Cu) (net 7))
 (via (at 145.923 138.303) (size 0.6858) (drill 0.3302) (layers F.Cu B.Cu) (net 7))
 (segment (start 145.923 138.303) (end 144.272 136.652) (width 0.3048) (layer F.Cu) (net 7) (status 20))
 (segment (start 144.272 136.652) (end 143.971 136.652) (width 0.3048) (layer F.Cu) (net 7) (status 30))
 (segment (start 147.193 139.573) (end 147.447 139.573) (width 0.3048) (layer F.Cu) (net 8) (status 30))
 (segment (start 147.447 139.573) (end 148.463 140.589) (width 0.3048) (layer F.Cu) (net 8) (status 10))
 (segment (start 147.955 143.383) (end 144.225 143.383) (width 0.3048) (layer F.Cu) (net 8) (status 20))
 (segment (start 148.463 142.875) (end 147.955 143.383) (width 0.3048) (layer F.Cu) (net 8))
 (segment (start 148.463 140.589) (end 148.463 142.875) (width 0.3048) (layer F.Cu) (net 8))
 (segment (start 144.225 143.383) (end 143.971 143.637) (width 0.3048) (layer F.Cu) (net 8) (status 30))
 (segment (start 148.463 138.303) (end 147.193 139.573) (width 0.3048) (layer F.Cu) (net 8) (status 20))
 (segment (start 150.368 134.744) (end 150.368 134.494) (width 0.3048) (layer F.Cu) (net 8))
 (segment (start 148.463 136.649) (end 150.368 134.744) (width 0.3048) (layer F.Cu) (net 8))
 (segment (start 148.463 138.303) (end 148.463 136.649) (width 0.3048) (layer F.Cu) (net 8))
 (segment (start 147.193 142.113) (end 146.003 142.113) (width 0.3048) (layer F.Cu) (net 9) (status 10))
 (segment (start 146.003 142.113) (end 143.971 140.081) (width 0.3048) (layer F.Cu) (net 9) (status 20))
 (via (at 145.288 139.192) (size 0.6858) (drill 0.3302) (layers F.Cu B.Cu) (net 9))
 (segment (start 143.971 140.081) (end 144.399 140.081) (width 0.3048) (layer F.Cu) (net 9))
 (segment (start 144.399 140.081) (end 145.288 139.192) (width 0.3048) (layer F.Cu) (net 9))
 (via (at 145.288 134.366) (size 0.6858) (drill 0.3302) (layers F.Cu B.Cu) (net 9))
 (segment (start 145.275299 134.378701) (end 145.288 134.366) (width 0.3048) (layer B.Cu) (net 9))
 (segment (start 145.275299 138.694366) (end 145.275299 134.378701) (width 0.3048) (layer B.Cu) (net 9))
 (segment (start 145.288 139.192) (end 145.288 138.707067) (width 0.3048) (layer B.Cu) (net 9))
 (segment (start 145.288 138.707067) (end 145.275299 138.694366) (width 0.3048) (layer B.Cu) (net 9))
 (segment (start 146.116 134.366) (end 146.624 133.858) (width 0.3048) (layer F.Cu) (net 9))
 (segment (start 145.288 134.366) (end 146.116 134.366) (width 0.3048) (layer F.Cu) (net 9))
 (segment (start 146.516642 130.438) (end 146.624 130.438) (width 0.3048) (layer F.Cu) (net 10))
 (segment (start 136.398 140.267081) (end 136.719919 140.589) (width 0.3048) (layer F.Cu) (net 10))
 (segment (start 136.398 129.495358) (end 136.398 140.267081) (width 0.3048) (layer F.Cu) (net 10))
 (segment (start 136.671159 129.222199) (end 136.398 129.495358) (width 0.3048) (layer F.Cu) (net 10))
 (segment (start 145.869801 129.283159) (end 145.808841 129.222199) (width 0.3048) (layer F.Cu) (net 10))
 (segment (start 136.719919 140.589) (end 137.922 140.589) (width 0.3048) (layer F.Cu) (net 10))
 (segment (start 145.869801 130.313601) (end 145.869801 129.283159) (width 0.3048) (layer F.Cu) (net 10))
 (segment (start 145.808841 129.222199) (end 136.671159 129.222199) (width 0.3048) (layer F.Cu) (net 10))
 (segment (start 145.9942 130.438) (end 145.869801 130.313601) (width 0.3048) (layer F.Cu) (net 10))
 (segment (start 146.624 130.438) (end 145.9942 130.438) (width 0.3048) (layer F.Cu) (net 10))
 (segment (start 143.571 144.5478) (end 143.3388 144.78) (width 0.3048) (layer B.Cu) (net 1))
 (segment (start 143.571 143.463) (end 143.571 144.5478) (width 0.3048) (layer B.Cu) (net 1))
 (segment (start 143.3388 144.78) (end 141.732 144.78) (width 0.3048) (layer B.Cu) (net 1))
 (segment (start 141.371 145.141) (end 141.371 146.177) (width 0.3048) (layer B.Cu) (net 1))
 (segment (start 141.732 144.78) (end 141.371 145.141) (width 0.3048) (layer B.Cu) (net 1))
 (segment (start 141.671 144.719) (end 141.732 144.78) (width 0.3048) (layer B.Cu) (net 1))
 (segment (start 141.671 143.463) (end 141.671 144.719) (width 0.3048) (layer B.Cu) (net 1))
 (via (at 141.304 146.177) (size 0.6858) (drill 0.3302) (layers F.Cu B.Cu) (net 1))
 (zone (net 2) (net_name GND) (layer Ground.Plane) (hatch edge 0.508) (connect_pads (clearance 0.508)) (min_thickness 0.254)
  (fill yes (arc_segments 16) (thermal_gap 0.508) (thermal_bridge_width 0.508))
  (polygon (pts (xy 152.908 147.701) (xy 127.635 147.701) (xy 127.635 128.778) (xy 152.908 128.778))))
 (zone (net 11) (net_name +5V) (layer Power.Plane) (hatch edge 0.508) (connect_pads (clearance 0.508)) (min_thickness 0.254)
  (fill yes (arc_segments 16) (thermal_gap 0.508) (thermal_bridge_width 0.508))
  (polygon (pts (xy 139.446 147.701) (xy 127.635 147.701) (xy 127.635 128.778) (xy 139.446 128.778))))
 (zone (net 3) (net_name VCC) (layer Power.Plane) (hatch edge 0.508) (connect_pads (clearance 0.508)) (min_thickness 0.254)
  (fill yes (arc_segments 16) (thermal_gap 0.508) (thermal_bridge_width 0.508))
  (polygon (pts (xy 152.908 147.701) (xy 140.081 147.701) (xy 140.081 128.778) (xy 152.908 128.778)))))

